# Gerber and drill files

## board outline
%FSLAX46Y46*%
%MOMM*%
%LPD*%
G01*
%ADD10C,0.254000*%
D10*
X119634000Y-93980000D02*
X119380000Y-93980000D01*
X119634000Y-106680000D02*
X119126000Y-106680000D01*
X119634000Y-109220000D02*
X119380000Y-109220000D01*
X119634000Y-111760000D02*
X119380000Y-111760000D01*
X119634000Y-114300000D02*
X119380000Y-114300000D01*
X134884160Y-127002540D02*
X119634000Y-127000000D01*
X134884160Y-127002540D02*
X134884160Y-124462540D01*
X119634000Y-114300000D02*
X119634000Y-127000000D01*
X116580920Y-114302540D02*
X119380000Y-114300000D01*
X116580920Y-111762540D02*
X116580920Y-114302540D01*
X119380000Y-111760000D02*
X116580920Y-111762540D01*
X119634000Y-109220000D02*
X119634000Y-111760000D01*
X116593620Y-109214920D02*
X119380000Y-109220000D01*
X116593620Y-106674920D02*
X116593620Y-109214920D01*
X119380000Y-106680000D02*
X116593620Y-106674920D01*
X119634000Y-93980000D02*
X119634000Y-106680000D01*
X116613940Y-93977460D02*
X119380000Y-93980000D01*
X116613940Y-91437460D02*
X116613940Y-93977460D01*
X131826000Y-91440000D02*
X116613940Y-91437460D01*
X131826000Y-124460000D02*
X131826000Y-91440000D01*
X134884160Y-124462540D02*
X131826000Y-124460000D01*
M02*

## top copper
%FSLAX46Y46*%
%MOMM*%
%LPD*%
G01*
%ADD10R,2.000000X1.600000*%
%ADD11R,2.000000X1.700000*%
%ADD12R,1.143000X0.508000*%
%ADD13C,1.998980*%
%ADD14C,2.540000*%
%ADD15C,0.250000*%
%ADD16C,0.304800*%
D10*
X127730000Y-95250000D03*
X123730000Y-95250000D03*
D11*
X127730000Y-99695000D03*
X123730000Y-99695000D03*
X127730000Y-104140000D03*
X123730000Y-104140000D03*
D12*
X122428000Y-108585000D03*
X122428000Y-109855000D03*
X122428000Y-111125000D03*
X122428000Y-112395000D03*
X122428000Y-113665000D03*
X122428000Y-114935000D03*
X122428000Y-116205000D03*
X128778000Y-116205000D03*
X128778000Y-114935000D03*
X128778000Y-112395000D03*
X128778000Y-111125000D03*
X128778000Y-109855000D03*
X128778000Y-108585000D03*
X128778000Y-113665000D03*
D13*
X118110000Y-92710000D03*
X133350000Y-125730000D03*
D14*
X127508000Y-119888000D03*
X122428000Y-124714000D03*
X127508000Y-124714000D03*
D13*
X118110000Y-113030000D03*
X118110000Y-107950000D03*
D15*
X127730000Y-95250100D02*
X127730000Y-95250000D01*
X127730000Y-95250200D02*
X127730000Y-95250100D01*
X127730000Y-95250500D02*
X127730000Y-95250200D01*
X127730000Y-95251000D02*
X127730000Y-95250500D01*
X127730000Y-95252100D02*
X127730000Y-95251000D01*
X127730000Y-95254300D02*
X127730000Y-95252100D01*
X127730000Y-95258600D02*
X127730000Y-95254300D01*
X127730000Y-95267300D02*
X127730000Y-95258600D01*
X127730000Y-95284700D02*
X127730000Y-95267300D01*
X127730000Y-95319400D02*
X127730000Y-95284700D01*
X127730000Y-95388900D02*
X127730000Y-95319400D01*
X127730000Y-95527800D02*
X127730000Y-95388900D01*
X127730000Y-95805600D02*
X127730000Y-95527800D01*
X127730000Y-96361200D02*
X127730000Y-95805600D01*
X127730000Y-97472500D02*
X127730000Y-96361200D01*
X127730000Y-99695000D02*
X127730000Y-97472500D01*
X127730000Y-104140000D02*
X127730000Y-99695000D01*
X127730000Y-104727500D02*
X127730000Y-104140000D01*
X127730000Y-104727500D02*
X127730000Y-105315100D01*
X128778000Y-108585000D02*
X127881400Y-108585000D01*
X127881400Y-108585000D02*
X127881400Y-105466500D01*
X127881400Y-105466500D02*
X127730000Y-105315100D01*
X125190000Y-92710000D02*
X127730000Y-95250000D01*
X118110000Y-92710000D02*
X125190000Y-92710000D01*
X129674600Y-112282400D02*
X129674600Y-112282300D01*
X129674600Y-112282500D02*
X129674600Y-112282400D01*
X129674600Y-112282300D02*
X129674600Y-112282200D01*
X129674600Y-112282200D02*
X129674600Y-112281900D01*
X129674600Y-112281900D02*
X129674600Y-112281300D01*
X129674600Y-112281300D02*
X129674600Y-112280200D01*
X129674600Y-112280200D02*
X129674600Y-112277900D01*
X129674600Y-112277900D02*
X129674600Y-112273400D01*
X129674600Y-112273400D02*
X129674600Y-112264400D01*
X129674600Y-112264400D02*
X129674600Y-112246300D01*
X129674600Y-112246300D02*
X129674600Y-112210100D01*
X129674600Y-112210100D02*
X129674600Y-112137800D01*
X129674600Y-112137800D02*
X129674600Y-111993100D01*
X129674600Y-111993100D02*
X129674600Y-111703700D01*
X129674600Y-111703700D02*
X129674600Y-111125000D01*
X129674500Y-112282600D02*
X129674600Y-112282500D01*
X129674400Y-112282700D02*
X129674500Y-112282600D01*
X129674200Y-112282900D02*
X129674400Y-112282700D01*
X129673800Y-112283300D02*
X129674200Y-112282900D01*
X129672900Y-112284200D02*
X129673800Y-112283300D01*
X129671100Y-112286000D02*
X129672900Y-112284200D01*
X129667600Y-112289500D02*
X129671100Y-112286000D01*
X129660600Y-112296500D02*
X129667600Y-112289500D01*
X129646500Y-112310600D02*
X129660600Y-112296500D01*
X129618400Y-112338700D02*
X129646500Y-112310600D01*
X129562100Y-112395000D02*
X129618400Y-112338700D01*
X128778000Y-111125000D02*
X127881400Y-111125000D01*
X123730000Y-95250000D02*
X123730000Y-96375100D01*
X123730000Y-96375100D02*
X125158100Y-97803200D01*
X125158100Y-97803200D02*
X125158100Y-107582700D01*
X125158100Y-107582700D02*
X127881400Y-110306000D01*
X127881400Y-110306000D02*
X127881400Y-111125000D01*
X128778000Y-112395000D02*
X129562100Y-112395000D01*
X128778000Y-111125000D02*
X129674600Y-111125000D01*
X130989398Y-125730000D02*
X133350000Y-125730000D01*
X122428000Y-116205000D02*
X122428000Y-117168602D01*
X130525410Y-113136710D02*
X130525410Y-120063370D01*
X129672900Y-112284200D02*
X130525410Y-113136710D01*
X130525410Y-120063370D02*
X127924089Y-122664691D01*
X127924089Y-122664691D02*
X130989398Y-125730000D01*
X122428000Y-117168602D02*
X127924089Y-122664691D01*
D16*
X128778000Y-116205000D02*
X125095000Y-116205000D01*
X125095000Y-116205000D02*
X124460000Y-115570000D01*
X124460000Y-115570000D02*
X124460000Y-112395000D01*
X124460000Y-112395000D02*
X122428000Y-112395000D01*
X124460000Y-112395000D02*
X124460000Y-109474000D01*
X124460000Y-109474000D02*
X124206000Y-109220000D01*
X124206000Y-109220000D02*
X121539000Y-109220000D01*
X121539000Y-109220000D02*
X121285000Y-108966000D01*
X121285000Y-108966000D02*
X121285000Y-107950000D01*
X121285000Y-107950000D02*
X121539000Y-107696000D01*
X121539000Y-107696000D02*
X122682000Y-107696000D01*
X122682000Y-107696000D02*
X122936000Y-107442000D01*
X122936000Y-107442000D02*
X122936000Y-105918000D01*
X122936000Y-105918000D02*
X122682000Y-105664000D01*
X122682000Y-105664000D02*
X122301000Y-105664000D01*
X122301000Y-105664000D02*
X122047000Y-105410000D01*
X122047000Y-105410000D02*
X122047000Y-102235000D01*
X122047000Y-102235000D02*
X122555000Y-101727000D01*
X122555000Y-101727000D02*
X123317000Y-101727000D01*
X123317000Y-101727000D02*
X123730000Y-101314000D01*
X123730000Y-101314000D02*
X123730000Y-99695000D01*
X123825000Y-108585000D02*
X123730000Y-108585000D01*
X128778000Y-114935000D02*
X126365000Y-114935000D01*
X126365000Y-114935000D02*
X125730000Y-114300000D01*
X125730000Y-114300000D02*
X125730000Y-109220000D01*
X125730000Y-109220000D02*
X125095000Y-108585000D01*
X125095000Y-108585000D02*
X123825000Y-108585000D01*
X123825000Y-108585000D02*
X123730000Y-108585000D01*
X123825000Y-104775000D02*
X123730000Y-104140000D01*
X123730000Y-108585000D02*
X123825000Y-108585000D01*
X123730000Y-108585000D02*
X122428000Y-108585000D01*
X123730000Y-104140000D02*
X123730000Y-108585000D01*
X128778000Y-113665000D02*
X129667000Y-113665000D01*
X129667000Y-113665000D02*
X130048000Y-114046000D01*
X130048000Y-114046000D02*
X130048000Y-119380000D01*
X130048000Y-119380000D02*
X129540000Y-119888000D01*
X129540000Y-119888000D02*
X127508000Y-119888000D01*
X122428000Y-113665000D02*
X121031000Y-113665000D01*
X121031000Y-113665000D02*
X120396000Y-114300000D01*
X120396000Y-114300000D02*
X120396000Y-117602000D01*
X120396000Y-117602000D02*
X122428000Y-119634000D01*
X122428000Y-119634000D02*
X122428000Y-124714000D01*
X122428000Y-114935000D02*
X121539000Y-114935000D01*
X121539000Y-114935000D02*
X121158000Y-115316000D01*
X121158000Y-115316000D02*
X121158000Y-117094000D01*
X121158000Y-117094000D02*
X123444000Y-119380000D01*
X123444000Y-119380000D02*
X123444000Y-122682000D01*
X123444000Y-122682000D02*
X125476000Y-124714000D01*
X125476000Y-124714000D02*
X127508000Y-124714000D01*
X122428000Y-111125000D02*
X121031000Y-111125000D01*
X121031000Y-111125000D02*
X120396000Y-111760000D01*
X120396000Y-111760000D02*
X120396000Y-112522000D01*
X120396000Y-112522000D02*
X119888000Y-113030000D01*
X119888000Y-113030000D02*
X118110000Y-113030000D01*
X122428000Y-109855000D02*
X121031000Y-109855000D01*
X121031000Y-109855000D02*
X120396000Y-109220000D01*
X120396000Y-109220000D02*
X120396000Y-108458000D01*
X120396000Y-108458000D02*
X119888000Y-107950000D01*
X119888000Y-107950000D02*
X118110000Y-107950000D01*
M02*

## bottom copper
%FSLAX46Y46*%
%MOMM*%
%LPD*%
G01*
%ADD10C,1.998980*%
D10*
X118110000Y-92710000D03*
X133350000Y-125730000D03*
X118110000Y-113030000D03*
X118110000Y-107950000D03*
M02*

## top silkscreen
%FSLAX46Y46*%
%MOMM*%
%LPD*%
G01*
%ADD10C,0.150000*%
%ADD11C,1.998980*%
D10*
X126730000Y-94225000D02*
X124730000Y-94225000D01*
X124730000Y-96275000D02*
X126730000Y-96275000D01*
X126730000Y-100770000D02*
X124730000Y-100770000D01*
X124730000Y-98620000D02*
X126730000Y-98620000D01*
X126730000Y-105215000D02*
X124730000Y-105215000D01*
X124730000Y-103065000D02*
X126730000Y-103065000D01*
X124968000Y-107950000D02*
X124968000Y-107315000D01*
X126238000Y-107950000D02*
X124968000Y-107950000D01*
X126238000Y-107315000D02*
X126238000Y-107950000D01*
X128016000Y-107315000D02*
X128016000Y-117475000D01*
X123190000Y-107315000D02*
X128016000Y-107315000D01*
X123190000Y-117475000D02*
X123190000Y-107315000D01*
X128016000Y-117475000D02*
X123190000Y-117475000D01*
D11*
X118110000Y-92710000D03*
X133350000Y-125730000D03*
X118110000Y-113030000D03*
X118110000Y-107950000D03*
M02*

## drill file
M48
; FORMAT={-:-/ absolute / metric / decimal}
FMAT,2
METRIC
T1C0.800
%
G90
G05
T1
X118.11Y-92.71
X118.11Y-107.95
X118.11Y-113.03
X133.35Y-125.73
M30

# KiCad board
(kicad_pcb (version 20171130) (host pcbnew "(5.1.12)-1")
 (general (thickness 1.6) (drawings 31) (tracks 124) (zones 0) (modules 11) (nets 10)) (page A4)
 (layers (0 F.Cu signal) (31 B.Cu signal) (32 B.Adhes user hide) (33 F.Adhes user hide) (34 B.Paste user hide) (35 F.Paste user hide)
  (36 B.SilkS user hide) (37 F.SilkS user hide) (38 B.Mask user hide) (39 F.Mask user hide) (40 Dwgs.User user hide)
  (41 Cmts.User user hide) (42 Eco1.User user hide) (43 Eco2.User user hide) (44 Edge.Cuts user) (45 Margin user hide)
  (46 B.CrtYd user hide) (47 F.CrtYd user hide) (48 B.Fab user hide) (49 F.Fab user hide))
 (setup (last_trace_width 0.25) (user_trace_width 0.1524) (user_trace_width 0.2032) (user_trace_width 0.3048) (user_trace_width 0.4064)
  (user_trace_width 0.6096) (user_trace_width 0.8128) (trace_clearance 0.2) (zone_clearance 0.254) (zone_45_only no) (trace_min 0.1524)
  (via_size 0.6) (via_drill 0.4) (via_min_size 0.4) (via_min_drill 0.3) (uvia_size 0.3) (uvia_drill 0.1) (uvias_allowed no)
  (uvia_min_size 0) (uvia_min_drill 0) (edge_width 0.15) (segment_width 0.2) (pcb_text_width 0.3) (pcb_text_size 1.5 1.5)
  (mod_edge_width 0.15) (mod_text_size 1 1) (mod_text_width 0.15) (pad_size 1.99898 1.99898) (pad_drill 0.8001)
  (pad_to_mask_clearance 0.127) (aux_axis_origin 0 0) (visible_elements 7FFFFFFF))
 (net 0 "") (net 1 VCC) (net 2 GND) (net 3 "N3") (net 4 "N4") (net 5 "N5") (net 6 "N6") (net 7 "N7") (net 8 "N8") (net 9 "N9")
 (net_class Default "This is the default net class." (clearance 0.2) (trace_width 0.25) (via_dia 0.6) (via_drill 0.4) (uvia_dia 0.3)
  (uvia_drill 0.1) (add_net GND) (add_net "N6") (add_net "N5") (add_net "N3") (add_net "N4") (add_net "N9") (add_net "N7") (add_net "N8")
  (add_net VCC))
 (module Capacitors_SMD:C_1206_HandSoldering (layer F.Cu) (at 125.73 95.25 180)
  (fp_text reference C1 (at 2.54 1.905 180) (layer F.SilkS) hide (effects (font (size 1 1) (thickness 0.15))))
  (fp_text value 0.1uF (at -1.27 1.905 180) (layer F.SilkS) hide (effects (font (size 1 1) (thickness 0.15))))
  (fp_line (start -1 1.025) (end 1 1.025) (layer F.SilkS) (width 0.15))
  (fp_line (start 1 -1.025) (end -1 -1.025) (layer F.SilkS) (width 0.15))
  (pad 1 smd rect (at -2 0 180) (size 2 1.6) (layers F.Cu F.Paste F.Mask) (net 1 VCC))
  (pad 2 smd rect (at 2 0 180) (size 2 1.6) (layers F.Cu F.Paste F.Mask) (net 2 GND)))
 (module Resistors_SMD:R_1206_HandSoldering (layer F.Cu) (at 125.73 99.695 180)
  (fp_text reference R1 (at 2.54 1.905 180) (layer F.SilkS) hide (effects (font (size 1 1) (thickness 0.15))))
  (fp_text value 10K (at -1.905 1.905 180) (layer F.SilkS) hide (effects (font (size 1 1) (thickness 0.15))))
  (fp_line (start -1 -1.075) (end 1 -1.075) (layer F.SilkS) (width 0.15))
  (fp_line (start 1 1.075) (end -1 1.075) (layer F.SilkS) (width 0.15))
  (pad 1 smd rect (at -2 0 180) (size 2 1.7) (layers F.Cu F.Paste F.Mask) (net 1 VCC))
  (pad 2 smd rect (at 2 0 180) (size 2 1.7) (layers F.Cu F.Paste F.Mask) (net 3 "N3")))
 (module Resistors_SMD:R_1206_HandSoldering (layer F.Cu) (at 125.73 104.14 180)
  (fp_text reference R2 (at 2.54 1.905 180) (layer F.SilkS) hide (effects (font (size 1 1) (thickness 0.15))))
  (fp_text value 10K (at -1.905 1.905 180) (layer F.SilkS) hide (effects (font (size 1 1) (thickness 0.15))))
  (fp_line (start -1 -1.075) (end 1 -1.075) (layer F.SilkS) (width 0.15))
  (fp_line (start 1 1.075) (end -1 1.075) (layer F.SilkS) (width 0.15))
  (pad 1 smd rect (at -2 0 180) (size 2 1.7) (layers F.Cu F.Paste F.Mask) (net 1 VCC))
  (pad 2 smd rect (at 2 0 180) (size 2 1.7) (layers F.Cu F.Paste F.Mask) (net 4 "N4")))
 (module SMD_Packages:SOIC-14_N (layer F.Cu) (at 125.73 112.395 270)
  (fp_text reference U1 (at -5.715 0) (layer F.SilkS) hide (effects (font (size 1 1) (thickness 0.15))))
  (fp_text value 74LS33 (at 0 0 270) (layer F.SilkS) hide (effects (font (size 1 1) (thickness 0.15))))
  (fp_line (start -4.445 0.762) (end -5.08 0.762) (layer F.SilkS) (width 0.15))
  (fp_line (start -4.445 -0.508) (end -4.445 0.762) (layer F.SilkS) (width 0.15))
  (fp_line (start -5.08 -0.508) (end -4.445 -0.508) (layer F.SilkS) (width 0.15))
  (fp_line (start -5.08 -2.286) (end 5.08 -2.286) (layer F.SilkS) (width 0.15))
  (fp_line (start -5.08 2.54) (end -5.08 -2.286) (layer F.SilkS) (width 0.15))
  (fp_line (start 5.08 2.54) (end -5.08 2.54) (layer F.SilkS) (width 0.15))
  (fp_line (start 5.08 -2.286) (end 5.08 2.54) (layer F.SilkS) (width 0.15))
  (pad 1 smd rect (at -3.81 3.302 270) (size 0.508 1.143) (layers F.Cu F.Paste F.Mask) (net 4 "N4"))
  (pad 2 smd rect (at -2.54 3.302 270) (size 0.508 1.143) (layers F.Cu F.Paste F.Mask) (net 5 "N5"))
  (pad 3 smd rect (at -1.27 3.302 270) (size 0.508 1.143) (layers F.Cu F.Paste F.Mask) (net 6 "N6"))
  (pad 4 smd rect (at 0 3.302 270) (size 0.508 1.143) (layers F.Cu F.Paste F.Mask) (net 3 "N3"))
  (pad 5 smd rect (at 1.27 3.302 270) (size 0.508 1.143) (layers F.Cu F.Paste F.Mask) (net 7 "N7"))
  (pad 6 smd rect (at 2.54 3.302 270) (size 0.508 1.143) (layers F.Cu F.Paste F.Mask) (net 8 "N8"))
  (pad 7 smd rect (at 3.81 3.302 270) (size 0.508 1.143) (layers F.Cu F.Paste F.Mask) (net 2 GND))
  (pad 8 smd rect (at 3.81 -3.048 270) (size 0.508 1.143) (layers F.Cu F.Paste F.Mask) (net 3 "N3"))
  (pad 9 smd rect (at 2.54 -3.048 270) (size 0.508 1.143) (layers F.Cu F.Paste F.Mask) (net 4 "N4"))
  (pad 11 smd rect (at 0 -3.048 270) (size 0.508 1.143) (layers F.Cu F.Paste F.Mask) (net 2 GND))
  (pad 12 smd rect (at -1.27 -3.048 270) (size 0.508 1.143) (layers F.Cu F.Paste F.Mask) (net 2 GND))
  (pad 13 smd rect (at -2.54 -3.048 270) (size 0.508 1.143) (layers F.Cu F.Paste F.Mask))
  (pad 14 smd rect (at -3.81 -3.048 270) (size 0.508 1.143) (layers F.Cu F.Paste F.Mask) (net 1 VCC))
  (pad 10 smd rect (at 1.27 -3.048 270) (size 0.508 1.143) (layers F.Cu F.Paste F.Mask) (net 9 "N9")))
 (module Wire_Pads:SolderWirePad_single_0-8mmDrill (layer F.Cu) (at 118.11 92.71 90)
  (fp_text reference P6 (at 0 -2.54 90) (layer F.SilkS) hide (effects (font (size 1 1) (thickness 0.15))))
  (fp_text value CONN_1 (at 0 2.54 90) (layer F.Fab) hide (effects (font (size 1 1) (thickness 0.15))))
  (pad 1 thru_hole circle (at 0 0 90) (size 1.99898 1.99898) (drill 0.8001) (layers *.Cu *.Mask F.SilkS) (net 1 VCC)))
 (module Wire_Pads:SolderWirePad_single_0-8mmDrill (layer F.Cu) (at 133.35 125.73 270)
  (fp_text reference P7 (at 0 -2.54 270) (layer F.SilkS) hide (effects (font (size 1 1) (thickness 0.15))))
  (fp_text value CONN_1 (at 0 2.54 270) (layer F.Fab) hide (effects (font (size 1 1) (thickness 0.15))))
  (pad 1 thru_hole circle (at 0 0 270) (size 1.99898 1.99898) (drill 0.8001) (layers *.Cu *.Mask F.SilkS) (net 2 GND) (zone_connect 2)))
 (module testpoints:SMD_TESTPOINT (layer F.Cu) (at 127.508 119.888)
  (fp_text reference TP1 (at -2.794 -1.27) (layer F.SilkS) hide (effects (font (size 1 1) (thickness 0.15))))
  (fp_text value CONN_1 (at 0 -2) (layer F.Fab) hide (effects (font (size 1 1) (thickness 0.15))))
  (pad 1 smd circle (at 0 0) (size 2.54 2.54) (layers F.Cu F.Paste F.Mask) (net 9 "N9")))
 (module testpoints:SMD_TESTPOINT (layer F.Cu) (at 122.428 124.714)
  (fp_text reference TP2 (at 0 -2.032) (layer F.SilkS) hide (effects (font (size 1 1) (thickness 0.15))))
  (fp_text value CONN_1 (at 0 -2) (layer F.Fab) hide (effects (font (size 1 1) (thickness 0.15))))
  (pad 1 smd circle (at 0 0) (size 2.54 2.54) (layers F.Cu F.Paste F.Mask) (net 7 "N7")))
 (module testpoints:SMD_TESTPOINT (layer F.Cu) (at 127.508 124.714)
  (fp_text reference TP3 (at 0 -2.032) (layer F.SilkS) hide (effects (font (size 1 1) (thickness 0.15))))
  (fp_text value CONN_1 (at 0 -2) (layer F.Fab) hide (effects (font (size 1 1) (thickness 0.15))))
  (pad 1 smd circle (at 0 0) (size 2.54 2.54) (layers F.Cu F.Paste F.Mask) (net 8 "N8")))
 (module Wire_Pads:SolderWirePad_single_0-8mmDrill (layer F.Cu) (at 118.11 113.03)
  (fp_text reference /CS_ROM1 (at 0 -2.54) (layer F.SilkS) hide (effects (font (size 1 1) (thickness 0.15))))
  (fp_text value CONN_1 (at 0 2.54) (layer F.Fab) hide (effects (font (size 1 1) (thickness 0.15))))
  (pad 1 thru_hole circle (at 0 0) (size 1.99898 1.99898) (drill 0.8001) (layers *.Cu *.Mask F.SilkS) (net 6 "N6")))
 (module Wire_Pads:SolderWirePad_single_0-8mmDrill (layer F.Cu) (at 118.11 107.95)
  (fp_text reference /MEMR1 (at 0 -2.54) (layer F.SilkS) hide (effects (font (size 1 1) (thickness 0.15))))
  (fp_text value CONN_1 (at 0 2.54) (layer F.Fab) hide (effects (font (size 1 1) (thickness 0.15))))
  (pad 1 thru_hole circle (at 0 0) (size 1.99898 1.99898) (drill 0.8001) (layers *.Cu *.Mask F.SilkS) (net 5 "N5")))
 (gr_line (start 119.634 93.98) (end 119.38 93.98) (angle 90) (layer Edge.Cuts) (width 0.254))
 (gr_line (start 119.634 106.68) (end 119.126 106.68) (angle 90) (layer Edge.Cuts) (width 0.254))
 (gr_line (start 119.634 109.22) (end 119.38 109.22) (angle 90) (layer Edge.Cuts) (width 0.254))
 (gr_line (start 119.634 111.76) (end 119.38 111.76) (angle 90) (layer Edge.Cuts) (width 0.254))
 (gr_line (start 119.634 114.3) (end 119.38 114.3) (angle 90) (layer Edge.Cuts) (width 0.254))
 (gr_line (start 134.88416 127.00254) (end 119.634 127) (angle 90) (layer Edge.Cuts) (width 0.254))
 (gr_line (start 134.88416 127.00254) (end 134.88416 124.46254) (angle 90) (layer Edge.Cuts) (width 0.254))
 (gr_line (start 119.634 114.3) (end 119.634 127) (angle 90) (layer Edge.Cuts) (width 0.254))
 (gr_line (start 116.58092 114.30254) (end 119.38 114.3) (angle 90) (layer Edge.Cuts) (width 0.254))
 (gr_line (start 116.58092 111.76254) (end 116.58092 114.30254) (angle 90) (layer Edge.Cuts) (width 0.254))
 (gr_line (start 119.38 111.76) (end 116.58092 111.76254) (angle 90) (layer Edge.Cuts) (width 0.254))
 (gr_line (start 119.634 109.22) (end 119.634 111.76) (angle 90) (layer Edge.Cuts) (width 0.254))
 (gr_line (start 116.59362 109.21492) (end 119.38 109.22) (angle 90) (layer Edge.Cuts) (width 0.254))
 (gr_line (start 116.59362 106.67492) (end 116.59362 109.21492) (angle 90) (layer Edge.Cuts) (width 0.254))
 (gr_line (start 119.38 106.68) (end 116.59362 106.67492) (angle 90) (layer Edge.Cuts) (width 0.254))
 (gr_line (start 119.634 93.98) (end 119.634 106.68) (angle 90) (layer Edge.Cuts) (width 0.254))
 (gr_line (start 116.61394 93.97746) (end 119.38 93.98) (angle 90) (layer Edge.Cuts) (width 0.254))
 (gr_line (start 116.61394 91.43746) (end 116.61394 93.97746) (angle 90) (layer Edge.Cuts) (width 0.254))
 (gr_line (start 131.826 91.44) (end 116.61394 91.43746) (angle 90) (layer Edge.Cuts) (width 0.254))
 (gr_line (start 131.826 124.46) (end 131.826 91.44) (angle 90) (layer Edge.Cuts) (width 0.254))
 (gr_line (start 134.88416 124.46254) (end 131.826 124.46) (angle 90) (layer Edge.Cuts) (width 0.254))
 (segment (start 127.73 95.2501) (end 127.73 95.25) (width 0.25) (layer F.Cu) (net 1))
 (segment (start 127.73 95.2502) (end 127.73 95.2501) (width 0.25) (layer F.Cu) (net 1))
 (segment (start 127.73 95.2505) (end 127.73 95.2502) (width 0.25) (layer F.Cu) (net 1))
 (segment (start 127.73 95.251) (end 127.73 95.2505) (width 0.25) (layer F.Cu) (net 1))
 (segment (start 127.73 95.2521) (end 127.73 95.251) (width 0.25) (layer F.Cu) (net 1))
 (segment (start 127.73 95.2543) (end 127.73 95.2521) (width 0.25) (layer F.Cu) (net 1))
 (segment (start 127.73 95.2586) (end 127.73 95.2543) (width 0.25) (layer F.Cu) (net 1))
 (segment (start 127.73 95.2673) (end 127.73 95.2586) (width 0.25) (layer F.Cu) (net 1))
 (segment (start 127.73 95.2847) (end 127.73 95.2673) (width 0.25) (layer F.Cu) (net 1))
 (segment (start 127.73 95.3194) (end 127.73 95.2847) (width 0.25) (layer F.Cu) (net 1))
 (segment (start 127.73 95.3889) (end 127.73 95.3194) (width 0.25) (layer F.Cu) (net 1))
 (segment (start 127.73 95.5278) (end 127.73 95.3889) (width 0.25) (layer F.Cu) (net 1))
 (segment (start 127.73 95.8056) (end 127.73 95.5278) (width 0.25) (layer F.Cu) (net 1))
 (segment (start 127.73 96.3612) (end 127.73 95.8056) (width 0.25) (layer F.Cu) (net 1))
 (segment (start 127.73 97.4725) (end 127.73 96.3612) (width 0.25) (layer F.Cu) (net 1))
 (segment (start 127.73 99.695) (end 127.73 97.4725) (width 0.25) (layer F.Cu) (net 1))
 (segment (start 127.73 104.14) (end 127.73 99.695) (width 0.25) (layer F.Cu) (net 1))
 (segment (start 127.73 104.7275) (end 127.73 104.14) (width 0.25) (layer F.Cu) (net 1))
 (segment (start 127.73 104.7275) (end 127.73 105.3151) (width 0.25) (layer F.Cu) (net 1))
 (segment (start 128.778 108.585) (end 127.8814 108.585) (width 0.25) (layer F.Cu) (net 1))
 (segment (start 127.8814 108.585) (end 127.8814 105.4665) (width 0.25) (layer F.Cu) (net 1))
 (segment (start 127.8814 105.4665) (end 127.73 105.3151) (width 0.25) (layer F.Cu) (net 1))
 (segment (start 125.19 92.71) (end 127.73 95.25) (width 0.25) (layer F.Cu) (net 1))
 (segment (start 118.11 92.71) (end 125.19 92.71) (width 0.25) (layer F.Cu) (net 1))
 (segment (start 129.6746 112.2824) (end 129.6746 112.2823) (width 0.25) (layer F.Cu) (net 2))
 (segment (start 129.6746 112.2825) (end 129.6746 112.2824) (width 0.25) (layer F.Cu) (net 2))
 (segment (start 129.6746 112.2823) (end 129.6746 112.2822) (width 0.25) (layer F.Cu) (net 2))
 (segment (start 129.6746 112.2822) (end 129.6746 112.2819) (width 0.25) (layer F.Cu) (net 2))
 (segment (start 129.6746 112.2819) (end 129.6746 112.2813) (width 0.25) (layer F.Cu) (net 2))
 (segment (start 129.6746 112.2813) (end 129.6746 112.2802) (width 0.25) (layer F.Cu) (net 2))
 (segment (start 129.6746 112.2802) (end 129.6746 112.2779) (width 0.25) (layer F.Cu) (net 2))
 (segment (start 129.6746 112.2779) (end 129.6746 112.2734) (width 0.25) (layer F.Cu) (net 2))
 (segment (start 129.6746 112.2734) (end 129.6746 112.2644) (width 0.25) (layer F.Cu) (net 2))
 (segment (start 129.6746 112.2644) (end 129.6746 112.2463) (width 0.25) (layer F.Cu) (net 2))
 (segment (start 129.6746 112.2463) (end 129.6746 112.2101) (width 0.25) (layer F.Cu) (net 2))
 (segment (start 129.6746 112.2101) (end 129.6746 112.1378) (width 0.25) (layer F.Cu) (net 2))
 (segment (start 129.6746 112.1378) (end 129.6746 111.9931) (width 0.25) (layer F.Cu) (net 2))
 (segment (start 129.6746 111.9931) (end 129.6746 111.7037) (width 0.25) (layer F.Cu) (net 2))
 (segment (start 129.6746 111.7037) (end 129.6746 111.125) (width 0.25) (layer F.Cu) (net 2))
 (segment (start 129.6745 112.2826) (end 129.6746 112.2825) (width 0.25) (layer F.Cu) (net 2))
 (segment (start 129.6744 112.2827) (end 129.6745 112.2826) (width 0.25) (layer F.Cu) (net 2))
 (segment (start 129.6742 112.2829) (end 129.6744 112.2827) (width 0.25) (layer F.Cu) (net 2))
 (segment (start 129.6738 112.2833) (end 129.6742 112.2829) (width 0.25) (layer F.Cu) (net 2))
 (segment (start 129.6729 112.2842) (end 129.6738 112.2833) (width 0.25) (layer F.Cu) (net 2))
 (segment (start 129.6711 112.286) (end 129.6729 112.2842) (width 0.25) (layer F.Cu) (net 2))
 (segment (start 129.6676 112.2895) (end 129.6711 112.286) (width 0.25) (layer F.Cu) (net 2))
 (segment (start 129.6606 112.2965) (end 129.6676 112.2895) (width 0.25) (layer F.Cu) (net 2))
 (segment (start 129.6465 112.3106) (end 129.6606 112.2965) (width 0.25) (layer F.Cu) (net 2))
 (segment (start 129.6184 112.3387) (end 129.6465 112.3106) (width 0.25) (layer F.Cu) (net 2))
 (segment (start 129.5621 112.395) (end 129.6184 112.3387) (width 0.25) (layer F.Cu) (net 2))
 (segment (start 128.778 111.125) (end 127.8814 111.125) (width 0.25) (layer F.Cu) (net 2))
 (segment (start 123.73 95.25) (end 123.73 96.3751) (width 0.25) (layer F.Cu) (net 2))
 (segment (start 123.73 96.3751) (end 125.1581 97.8032) (width 0.25) (layer F.Cu) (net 2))
 (segment (start 125.1581 97.8032) (end 125.1581 107.5827) (width 0.25) (layer F.Cu) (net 2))
 (segment (start 125.1581 107.5827) (end 127.8814 110.306) (width 0.25) (layer F.Cu) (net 2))
 (segment (start 127.8814 110.306) (end 127.8814 111.125) (width 0.25) (layer F.Cu) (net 2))
 (segment (start 128.778 112.395) (end 129.5621 112.395) (width 0.25) (layer F.Cu) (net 2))
 (segment (start 128.778 111.125) (end 129.6746 111.125) (width 0.25) (layer F.Cu) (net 2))
 (segment (start 130.989398 125.73) (end 133.35 125.73) (width 0.25) (layer F.Cu) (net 2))
 (segment (start 122.428 116.205) (end 122.428 117.168602) (width 0.25) (layer F.Cu) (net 2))
 (segment (start 130.52541 113.13671) (end 130.52541 120.06337) (width 0.25) (layer F.Cu) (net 2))
 (segment (start 129.6729 112.2842) (end 130.52541 113.13671) (width 0.25) (layer F.Cu) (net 2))
 (segment (start 130.52541 120.06337) (end 127.924089 122.664691) (width 0.25) (layer F.Cu) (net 2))
 (segment (start 127.924089 122.664691) (end 130.989398 125.73) (width 0.25) (layer F.Cu) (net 2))
 (segment (start 122.428 117.168602) (end 127.924089 122.664691) (width 0.25) (layer F.Cu) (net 2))
 (segment (start 128.778 116.205) (end 125.095 116.205) (width 0.3048) (layer F.Cu) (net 3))
 (segment (start 125.095 116.205) (end 124.46 115.57) (width 0.3048) (layer F.Cu) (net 3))
 (segment (start 124.46 115.57) (end 124.46 112.395) (width 0.3048) (layer F.Cu) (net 3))
 (segment (start 124.46 112.395) (end 122.428 112.395) (width 0.3048) (layer F.Cu) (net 3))
 (segment (start 124.46 112.395) (end 124.46 109.474) (width 0.3048) (layer F.Cu) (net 3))
 (segment (start 124.46 109.474) (end 124.206 109.22) (width 0.3048) (layer F.Cu) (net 3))
 (segment (start 124.206 109.22) (end 121.539 109.22) (width 0.3048) (layer F.Cu) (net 3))
 (segment (start 121.539 109.22) (end 121.285 108.966) (width 0.3048) (layer F.Cu) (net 3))
 (segment (start 121.285 108.966) (end 121.285 107.95) (width 0.3048) (layer F.Cu) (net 3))
 (segment (start 121.285 107.95) (end 121.539 107.696) (width 0.3048) (layer F.Cu) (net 3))
 (segment (start 121.539 107.696) (end 122.682 107.696) (width 0.3048) (layer F.Cu) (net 3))
 (segment (start 122.682 107.696) (end 122.936 107.442) (width 0.3048) (layer F.Cu) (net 3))
 (segment (start 122.936 107.442) (end 122.936 105.918) (width 0.3048) (layer F.Cu) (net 3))
 (segment (start 122.936 105.918) (end 122.682 105.664) (width 0.3048) (layer F.Cu) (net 3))
 (segment (start 122.682 105.664) (end 122.301 105.664) (width 0.3048) (layer F.Cu) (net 3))
 (segment (start 122.301 105.664) (end 122.047 105.41) (width 0.3048) (layer F.Cu) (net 3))
 (segment (start 122.047 105.41) (end 122.047 102.235) (width 0.3048) (layer F.Cu) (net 3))
 (segment (start 122.047 102.235) (end 122.555 101.727) (width 0.3048) (layer F.Cu) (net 3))
 (segment (start 122.555 101.727) (end 123.317 101.727) (width 0.3048) (layer F.Cu) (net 3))
 (segment (start 123.317 101.727) (end 123.73 101.314) (width 0.3048) (layer F.Cu) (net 3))
 (segment (start 123.73 101.314) (end 123.73 99.695) (width 0.3048) (layer F.Cu) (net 3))
 (segment (start 123.825 108.585) (end 123.73 108.585) (width 0.3048) (layer F.Cu) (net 4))
 (segment (start 128.778 114.935) (end 126.365 114.935) (width 0.3048) (layer F.Cu) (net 4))
 (segment (start 126.365 114.935) (end 125.73 114.3) (width 0.3048) (layer F.Cu) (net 4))
 (segment (start 125.73 114.3) (end 125.73 109.22) (width 0.3048) (layer F.Cu) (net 4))
 (segment (start 125.73 109.22) (end 125.095 108.585) (width 0.3048) (layer F.Cu) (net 4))
 (segment (start 125.095 108.585) (end 123.825 108.585) (width 0.3048) (layer F.Cu) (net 4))
 (segment (start 123.825 108.585) (end 123.73 108.585) (width 0.3048) (layer F.Cu) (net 4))
 (segment (start 123.825 104.775) (end 123.73 104.14) (width 0.3048) (layer F.Cu) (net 4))
 (segment (start 123.73 108.585) (end 123.825 108.585) (width 0.3048) (layer F.Cu) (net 4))
 (segment (start 123.73 108.585) (end 122.428 108.585) (width 0.3048) (layer F.Cu) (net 4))
 (segment (start 123.73 104.14) (end 123.73 108.585) (width 0.3048) (layer F.Cu) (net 4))
 (segment (start 128.778 113.665) (end 129.667 113.665) (width 0.3048) (layer F.Cu) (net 9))
 (segment (start 129.667 113.665) (end 130.048 114.046) (width 0.3048) (layer F.Cu) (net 9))
 (segment (start 130.048 114.046) (end 130.048 119.38) (width 0.3048) (layer F.Cu) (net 9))
 (segment (start 130.048 119.38) (end 129.54 119.888) (width 0.3048) (layer F.Cu) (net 9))
 (segment (start 129.54 119.888) (end 127.508 119.888) (width 0.3048) (layer F.Cu) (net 9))
 (segment (start 122.428 113.665) (end 121.031 113.665) (width 0.3048) (layer F.Cu) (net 7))
 (segment (start 121.031 113.665) (end 120.396 114.3) (width 0.3048) (layer F.Cu) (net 7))
 (segment (start 120.396 114.3) (end 120.396 117.602) (width 0.3048) (layer F.Cu) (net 7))
 (segment (start 120.396 117.602) (end 122.428 119.634) (width 0.3048) (layer F.Cu) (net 7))
 (segment (start 122.428 119.634) (end 122.428 124.714) (width 0.3048) (layer F.Cu) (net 7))
 (segment (start 122.428 114.935) (end 121.539 114.935) (width 0.3048) (layer F.Cu) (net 8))
 (segment (start 121.539 114.935) (end 121.158 115.316) (width 0.3048) (layer F.Cu) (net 8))
 (segment (start 121.158 115.316) (end 121.158 117.094) (width 0.3048) (layer F.Cu) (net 8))
 (segment (start 121.158 117.094) (end 123.444 119.38) (width 0.3048) (layer F.Cu) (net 8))
 (segment (start 123.444 119.38) (end 123.444 122.682) (width 0.3048) (layer F.Cu) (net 8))
 (segment (start 123.444 122.682) (end 125.476 124.714) (width 0.3048) (layer F.Cu) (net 8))
 (segment (start 125.476 124.714) (end 127.508 124.714) (width 0.3048) (layer F.Cu) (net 8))
 (segment (start 122.428 111.125) (end 121.031 111.125) (width 0.3048) (layer F.Cu) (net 6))
 (segment (start 121.031 111.125) (end 120.396 111.76) (width 0.3048) (layer F.Cu) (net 6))
 (segment (start 120.396 111.76) (end 120.396 112.522) (width 0.3048) (layer F.Cu) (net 6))
 (segment (start 120.396 112.522) (end 119.888 113.03) (width 0.3048) (layer F.Cu) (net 6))
 (segment (start 119.888 113.03) (end 118.11 113.03) (width 0.3048) (layer F.Cu) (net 6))
 (segment (start 122.428 109.855) (end 121.031 109.855) (width 0.3048) (layer F.Cu) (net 5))
 (segment (start 121.031 109.855) (end 120.396 109.22) (width 0.3048) (layer F.Cu) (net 5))
 (segment (start 120.396 109.22) (end 120.396 108.458) (width 0.3048) (layer F.Cu) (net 5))
 (segment (start 120.396 108.458) (end 119.888 107.95) (width 0.3048) (layer F.Cu) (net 5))
 (segment (start 119.888 107.95) (end 118.11 107.95) (width 0.3048) (layer F.Cu) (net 5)))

